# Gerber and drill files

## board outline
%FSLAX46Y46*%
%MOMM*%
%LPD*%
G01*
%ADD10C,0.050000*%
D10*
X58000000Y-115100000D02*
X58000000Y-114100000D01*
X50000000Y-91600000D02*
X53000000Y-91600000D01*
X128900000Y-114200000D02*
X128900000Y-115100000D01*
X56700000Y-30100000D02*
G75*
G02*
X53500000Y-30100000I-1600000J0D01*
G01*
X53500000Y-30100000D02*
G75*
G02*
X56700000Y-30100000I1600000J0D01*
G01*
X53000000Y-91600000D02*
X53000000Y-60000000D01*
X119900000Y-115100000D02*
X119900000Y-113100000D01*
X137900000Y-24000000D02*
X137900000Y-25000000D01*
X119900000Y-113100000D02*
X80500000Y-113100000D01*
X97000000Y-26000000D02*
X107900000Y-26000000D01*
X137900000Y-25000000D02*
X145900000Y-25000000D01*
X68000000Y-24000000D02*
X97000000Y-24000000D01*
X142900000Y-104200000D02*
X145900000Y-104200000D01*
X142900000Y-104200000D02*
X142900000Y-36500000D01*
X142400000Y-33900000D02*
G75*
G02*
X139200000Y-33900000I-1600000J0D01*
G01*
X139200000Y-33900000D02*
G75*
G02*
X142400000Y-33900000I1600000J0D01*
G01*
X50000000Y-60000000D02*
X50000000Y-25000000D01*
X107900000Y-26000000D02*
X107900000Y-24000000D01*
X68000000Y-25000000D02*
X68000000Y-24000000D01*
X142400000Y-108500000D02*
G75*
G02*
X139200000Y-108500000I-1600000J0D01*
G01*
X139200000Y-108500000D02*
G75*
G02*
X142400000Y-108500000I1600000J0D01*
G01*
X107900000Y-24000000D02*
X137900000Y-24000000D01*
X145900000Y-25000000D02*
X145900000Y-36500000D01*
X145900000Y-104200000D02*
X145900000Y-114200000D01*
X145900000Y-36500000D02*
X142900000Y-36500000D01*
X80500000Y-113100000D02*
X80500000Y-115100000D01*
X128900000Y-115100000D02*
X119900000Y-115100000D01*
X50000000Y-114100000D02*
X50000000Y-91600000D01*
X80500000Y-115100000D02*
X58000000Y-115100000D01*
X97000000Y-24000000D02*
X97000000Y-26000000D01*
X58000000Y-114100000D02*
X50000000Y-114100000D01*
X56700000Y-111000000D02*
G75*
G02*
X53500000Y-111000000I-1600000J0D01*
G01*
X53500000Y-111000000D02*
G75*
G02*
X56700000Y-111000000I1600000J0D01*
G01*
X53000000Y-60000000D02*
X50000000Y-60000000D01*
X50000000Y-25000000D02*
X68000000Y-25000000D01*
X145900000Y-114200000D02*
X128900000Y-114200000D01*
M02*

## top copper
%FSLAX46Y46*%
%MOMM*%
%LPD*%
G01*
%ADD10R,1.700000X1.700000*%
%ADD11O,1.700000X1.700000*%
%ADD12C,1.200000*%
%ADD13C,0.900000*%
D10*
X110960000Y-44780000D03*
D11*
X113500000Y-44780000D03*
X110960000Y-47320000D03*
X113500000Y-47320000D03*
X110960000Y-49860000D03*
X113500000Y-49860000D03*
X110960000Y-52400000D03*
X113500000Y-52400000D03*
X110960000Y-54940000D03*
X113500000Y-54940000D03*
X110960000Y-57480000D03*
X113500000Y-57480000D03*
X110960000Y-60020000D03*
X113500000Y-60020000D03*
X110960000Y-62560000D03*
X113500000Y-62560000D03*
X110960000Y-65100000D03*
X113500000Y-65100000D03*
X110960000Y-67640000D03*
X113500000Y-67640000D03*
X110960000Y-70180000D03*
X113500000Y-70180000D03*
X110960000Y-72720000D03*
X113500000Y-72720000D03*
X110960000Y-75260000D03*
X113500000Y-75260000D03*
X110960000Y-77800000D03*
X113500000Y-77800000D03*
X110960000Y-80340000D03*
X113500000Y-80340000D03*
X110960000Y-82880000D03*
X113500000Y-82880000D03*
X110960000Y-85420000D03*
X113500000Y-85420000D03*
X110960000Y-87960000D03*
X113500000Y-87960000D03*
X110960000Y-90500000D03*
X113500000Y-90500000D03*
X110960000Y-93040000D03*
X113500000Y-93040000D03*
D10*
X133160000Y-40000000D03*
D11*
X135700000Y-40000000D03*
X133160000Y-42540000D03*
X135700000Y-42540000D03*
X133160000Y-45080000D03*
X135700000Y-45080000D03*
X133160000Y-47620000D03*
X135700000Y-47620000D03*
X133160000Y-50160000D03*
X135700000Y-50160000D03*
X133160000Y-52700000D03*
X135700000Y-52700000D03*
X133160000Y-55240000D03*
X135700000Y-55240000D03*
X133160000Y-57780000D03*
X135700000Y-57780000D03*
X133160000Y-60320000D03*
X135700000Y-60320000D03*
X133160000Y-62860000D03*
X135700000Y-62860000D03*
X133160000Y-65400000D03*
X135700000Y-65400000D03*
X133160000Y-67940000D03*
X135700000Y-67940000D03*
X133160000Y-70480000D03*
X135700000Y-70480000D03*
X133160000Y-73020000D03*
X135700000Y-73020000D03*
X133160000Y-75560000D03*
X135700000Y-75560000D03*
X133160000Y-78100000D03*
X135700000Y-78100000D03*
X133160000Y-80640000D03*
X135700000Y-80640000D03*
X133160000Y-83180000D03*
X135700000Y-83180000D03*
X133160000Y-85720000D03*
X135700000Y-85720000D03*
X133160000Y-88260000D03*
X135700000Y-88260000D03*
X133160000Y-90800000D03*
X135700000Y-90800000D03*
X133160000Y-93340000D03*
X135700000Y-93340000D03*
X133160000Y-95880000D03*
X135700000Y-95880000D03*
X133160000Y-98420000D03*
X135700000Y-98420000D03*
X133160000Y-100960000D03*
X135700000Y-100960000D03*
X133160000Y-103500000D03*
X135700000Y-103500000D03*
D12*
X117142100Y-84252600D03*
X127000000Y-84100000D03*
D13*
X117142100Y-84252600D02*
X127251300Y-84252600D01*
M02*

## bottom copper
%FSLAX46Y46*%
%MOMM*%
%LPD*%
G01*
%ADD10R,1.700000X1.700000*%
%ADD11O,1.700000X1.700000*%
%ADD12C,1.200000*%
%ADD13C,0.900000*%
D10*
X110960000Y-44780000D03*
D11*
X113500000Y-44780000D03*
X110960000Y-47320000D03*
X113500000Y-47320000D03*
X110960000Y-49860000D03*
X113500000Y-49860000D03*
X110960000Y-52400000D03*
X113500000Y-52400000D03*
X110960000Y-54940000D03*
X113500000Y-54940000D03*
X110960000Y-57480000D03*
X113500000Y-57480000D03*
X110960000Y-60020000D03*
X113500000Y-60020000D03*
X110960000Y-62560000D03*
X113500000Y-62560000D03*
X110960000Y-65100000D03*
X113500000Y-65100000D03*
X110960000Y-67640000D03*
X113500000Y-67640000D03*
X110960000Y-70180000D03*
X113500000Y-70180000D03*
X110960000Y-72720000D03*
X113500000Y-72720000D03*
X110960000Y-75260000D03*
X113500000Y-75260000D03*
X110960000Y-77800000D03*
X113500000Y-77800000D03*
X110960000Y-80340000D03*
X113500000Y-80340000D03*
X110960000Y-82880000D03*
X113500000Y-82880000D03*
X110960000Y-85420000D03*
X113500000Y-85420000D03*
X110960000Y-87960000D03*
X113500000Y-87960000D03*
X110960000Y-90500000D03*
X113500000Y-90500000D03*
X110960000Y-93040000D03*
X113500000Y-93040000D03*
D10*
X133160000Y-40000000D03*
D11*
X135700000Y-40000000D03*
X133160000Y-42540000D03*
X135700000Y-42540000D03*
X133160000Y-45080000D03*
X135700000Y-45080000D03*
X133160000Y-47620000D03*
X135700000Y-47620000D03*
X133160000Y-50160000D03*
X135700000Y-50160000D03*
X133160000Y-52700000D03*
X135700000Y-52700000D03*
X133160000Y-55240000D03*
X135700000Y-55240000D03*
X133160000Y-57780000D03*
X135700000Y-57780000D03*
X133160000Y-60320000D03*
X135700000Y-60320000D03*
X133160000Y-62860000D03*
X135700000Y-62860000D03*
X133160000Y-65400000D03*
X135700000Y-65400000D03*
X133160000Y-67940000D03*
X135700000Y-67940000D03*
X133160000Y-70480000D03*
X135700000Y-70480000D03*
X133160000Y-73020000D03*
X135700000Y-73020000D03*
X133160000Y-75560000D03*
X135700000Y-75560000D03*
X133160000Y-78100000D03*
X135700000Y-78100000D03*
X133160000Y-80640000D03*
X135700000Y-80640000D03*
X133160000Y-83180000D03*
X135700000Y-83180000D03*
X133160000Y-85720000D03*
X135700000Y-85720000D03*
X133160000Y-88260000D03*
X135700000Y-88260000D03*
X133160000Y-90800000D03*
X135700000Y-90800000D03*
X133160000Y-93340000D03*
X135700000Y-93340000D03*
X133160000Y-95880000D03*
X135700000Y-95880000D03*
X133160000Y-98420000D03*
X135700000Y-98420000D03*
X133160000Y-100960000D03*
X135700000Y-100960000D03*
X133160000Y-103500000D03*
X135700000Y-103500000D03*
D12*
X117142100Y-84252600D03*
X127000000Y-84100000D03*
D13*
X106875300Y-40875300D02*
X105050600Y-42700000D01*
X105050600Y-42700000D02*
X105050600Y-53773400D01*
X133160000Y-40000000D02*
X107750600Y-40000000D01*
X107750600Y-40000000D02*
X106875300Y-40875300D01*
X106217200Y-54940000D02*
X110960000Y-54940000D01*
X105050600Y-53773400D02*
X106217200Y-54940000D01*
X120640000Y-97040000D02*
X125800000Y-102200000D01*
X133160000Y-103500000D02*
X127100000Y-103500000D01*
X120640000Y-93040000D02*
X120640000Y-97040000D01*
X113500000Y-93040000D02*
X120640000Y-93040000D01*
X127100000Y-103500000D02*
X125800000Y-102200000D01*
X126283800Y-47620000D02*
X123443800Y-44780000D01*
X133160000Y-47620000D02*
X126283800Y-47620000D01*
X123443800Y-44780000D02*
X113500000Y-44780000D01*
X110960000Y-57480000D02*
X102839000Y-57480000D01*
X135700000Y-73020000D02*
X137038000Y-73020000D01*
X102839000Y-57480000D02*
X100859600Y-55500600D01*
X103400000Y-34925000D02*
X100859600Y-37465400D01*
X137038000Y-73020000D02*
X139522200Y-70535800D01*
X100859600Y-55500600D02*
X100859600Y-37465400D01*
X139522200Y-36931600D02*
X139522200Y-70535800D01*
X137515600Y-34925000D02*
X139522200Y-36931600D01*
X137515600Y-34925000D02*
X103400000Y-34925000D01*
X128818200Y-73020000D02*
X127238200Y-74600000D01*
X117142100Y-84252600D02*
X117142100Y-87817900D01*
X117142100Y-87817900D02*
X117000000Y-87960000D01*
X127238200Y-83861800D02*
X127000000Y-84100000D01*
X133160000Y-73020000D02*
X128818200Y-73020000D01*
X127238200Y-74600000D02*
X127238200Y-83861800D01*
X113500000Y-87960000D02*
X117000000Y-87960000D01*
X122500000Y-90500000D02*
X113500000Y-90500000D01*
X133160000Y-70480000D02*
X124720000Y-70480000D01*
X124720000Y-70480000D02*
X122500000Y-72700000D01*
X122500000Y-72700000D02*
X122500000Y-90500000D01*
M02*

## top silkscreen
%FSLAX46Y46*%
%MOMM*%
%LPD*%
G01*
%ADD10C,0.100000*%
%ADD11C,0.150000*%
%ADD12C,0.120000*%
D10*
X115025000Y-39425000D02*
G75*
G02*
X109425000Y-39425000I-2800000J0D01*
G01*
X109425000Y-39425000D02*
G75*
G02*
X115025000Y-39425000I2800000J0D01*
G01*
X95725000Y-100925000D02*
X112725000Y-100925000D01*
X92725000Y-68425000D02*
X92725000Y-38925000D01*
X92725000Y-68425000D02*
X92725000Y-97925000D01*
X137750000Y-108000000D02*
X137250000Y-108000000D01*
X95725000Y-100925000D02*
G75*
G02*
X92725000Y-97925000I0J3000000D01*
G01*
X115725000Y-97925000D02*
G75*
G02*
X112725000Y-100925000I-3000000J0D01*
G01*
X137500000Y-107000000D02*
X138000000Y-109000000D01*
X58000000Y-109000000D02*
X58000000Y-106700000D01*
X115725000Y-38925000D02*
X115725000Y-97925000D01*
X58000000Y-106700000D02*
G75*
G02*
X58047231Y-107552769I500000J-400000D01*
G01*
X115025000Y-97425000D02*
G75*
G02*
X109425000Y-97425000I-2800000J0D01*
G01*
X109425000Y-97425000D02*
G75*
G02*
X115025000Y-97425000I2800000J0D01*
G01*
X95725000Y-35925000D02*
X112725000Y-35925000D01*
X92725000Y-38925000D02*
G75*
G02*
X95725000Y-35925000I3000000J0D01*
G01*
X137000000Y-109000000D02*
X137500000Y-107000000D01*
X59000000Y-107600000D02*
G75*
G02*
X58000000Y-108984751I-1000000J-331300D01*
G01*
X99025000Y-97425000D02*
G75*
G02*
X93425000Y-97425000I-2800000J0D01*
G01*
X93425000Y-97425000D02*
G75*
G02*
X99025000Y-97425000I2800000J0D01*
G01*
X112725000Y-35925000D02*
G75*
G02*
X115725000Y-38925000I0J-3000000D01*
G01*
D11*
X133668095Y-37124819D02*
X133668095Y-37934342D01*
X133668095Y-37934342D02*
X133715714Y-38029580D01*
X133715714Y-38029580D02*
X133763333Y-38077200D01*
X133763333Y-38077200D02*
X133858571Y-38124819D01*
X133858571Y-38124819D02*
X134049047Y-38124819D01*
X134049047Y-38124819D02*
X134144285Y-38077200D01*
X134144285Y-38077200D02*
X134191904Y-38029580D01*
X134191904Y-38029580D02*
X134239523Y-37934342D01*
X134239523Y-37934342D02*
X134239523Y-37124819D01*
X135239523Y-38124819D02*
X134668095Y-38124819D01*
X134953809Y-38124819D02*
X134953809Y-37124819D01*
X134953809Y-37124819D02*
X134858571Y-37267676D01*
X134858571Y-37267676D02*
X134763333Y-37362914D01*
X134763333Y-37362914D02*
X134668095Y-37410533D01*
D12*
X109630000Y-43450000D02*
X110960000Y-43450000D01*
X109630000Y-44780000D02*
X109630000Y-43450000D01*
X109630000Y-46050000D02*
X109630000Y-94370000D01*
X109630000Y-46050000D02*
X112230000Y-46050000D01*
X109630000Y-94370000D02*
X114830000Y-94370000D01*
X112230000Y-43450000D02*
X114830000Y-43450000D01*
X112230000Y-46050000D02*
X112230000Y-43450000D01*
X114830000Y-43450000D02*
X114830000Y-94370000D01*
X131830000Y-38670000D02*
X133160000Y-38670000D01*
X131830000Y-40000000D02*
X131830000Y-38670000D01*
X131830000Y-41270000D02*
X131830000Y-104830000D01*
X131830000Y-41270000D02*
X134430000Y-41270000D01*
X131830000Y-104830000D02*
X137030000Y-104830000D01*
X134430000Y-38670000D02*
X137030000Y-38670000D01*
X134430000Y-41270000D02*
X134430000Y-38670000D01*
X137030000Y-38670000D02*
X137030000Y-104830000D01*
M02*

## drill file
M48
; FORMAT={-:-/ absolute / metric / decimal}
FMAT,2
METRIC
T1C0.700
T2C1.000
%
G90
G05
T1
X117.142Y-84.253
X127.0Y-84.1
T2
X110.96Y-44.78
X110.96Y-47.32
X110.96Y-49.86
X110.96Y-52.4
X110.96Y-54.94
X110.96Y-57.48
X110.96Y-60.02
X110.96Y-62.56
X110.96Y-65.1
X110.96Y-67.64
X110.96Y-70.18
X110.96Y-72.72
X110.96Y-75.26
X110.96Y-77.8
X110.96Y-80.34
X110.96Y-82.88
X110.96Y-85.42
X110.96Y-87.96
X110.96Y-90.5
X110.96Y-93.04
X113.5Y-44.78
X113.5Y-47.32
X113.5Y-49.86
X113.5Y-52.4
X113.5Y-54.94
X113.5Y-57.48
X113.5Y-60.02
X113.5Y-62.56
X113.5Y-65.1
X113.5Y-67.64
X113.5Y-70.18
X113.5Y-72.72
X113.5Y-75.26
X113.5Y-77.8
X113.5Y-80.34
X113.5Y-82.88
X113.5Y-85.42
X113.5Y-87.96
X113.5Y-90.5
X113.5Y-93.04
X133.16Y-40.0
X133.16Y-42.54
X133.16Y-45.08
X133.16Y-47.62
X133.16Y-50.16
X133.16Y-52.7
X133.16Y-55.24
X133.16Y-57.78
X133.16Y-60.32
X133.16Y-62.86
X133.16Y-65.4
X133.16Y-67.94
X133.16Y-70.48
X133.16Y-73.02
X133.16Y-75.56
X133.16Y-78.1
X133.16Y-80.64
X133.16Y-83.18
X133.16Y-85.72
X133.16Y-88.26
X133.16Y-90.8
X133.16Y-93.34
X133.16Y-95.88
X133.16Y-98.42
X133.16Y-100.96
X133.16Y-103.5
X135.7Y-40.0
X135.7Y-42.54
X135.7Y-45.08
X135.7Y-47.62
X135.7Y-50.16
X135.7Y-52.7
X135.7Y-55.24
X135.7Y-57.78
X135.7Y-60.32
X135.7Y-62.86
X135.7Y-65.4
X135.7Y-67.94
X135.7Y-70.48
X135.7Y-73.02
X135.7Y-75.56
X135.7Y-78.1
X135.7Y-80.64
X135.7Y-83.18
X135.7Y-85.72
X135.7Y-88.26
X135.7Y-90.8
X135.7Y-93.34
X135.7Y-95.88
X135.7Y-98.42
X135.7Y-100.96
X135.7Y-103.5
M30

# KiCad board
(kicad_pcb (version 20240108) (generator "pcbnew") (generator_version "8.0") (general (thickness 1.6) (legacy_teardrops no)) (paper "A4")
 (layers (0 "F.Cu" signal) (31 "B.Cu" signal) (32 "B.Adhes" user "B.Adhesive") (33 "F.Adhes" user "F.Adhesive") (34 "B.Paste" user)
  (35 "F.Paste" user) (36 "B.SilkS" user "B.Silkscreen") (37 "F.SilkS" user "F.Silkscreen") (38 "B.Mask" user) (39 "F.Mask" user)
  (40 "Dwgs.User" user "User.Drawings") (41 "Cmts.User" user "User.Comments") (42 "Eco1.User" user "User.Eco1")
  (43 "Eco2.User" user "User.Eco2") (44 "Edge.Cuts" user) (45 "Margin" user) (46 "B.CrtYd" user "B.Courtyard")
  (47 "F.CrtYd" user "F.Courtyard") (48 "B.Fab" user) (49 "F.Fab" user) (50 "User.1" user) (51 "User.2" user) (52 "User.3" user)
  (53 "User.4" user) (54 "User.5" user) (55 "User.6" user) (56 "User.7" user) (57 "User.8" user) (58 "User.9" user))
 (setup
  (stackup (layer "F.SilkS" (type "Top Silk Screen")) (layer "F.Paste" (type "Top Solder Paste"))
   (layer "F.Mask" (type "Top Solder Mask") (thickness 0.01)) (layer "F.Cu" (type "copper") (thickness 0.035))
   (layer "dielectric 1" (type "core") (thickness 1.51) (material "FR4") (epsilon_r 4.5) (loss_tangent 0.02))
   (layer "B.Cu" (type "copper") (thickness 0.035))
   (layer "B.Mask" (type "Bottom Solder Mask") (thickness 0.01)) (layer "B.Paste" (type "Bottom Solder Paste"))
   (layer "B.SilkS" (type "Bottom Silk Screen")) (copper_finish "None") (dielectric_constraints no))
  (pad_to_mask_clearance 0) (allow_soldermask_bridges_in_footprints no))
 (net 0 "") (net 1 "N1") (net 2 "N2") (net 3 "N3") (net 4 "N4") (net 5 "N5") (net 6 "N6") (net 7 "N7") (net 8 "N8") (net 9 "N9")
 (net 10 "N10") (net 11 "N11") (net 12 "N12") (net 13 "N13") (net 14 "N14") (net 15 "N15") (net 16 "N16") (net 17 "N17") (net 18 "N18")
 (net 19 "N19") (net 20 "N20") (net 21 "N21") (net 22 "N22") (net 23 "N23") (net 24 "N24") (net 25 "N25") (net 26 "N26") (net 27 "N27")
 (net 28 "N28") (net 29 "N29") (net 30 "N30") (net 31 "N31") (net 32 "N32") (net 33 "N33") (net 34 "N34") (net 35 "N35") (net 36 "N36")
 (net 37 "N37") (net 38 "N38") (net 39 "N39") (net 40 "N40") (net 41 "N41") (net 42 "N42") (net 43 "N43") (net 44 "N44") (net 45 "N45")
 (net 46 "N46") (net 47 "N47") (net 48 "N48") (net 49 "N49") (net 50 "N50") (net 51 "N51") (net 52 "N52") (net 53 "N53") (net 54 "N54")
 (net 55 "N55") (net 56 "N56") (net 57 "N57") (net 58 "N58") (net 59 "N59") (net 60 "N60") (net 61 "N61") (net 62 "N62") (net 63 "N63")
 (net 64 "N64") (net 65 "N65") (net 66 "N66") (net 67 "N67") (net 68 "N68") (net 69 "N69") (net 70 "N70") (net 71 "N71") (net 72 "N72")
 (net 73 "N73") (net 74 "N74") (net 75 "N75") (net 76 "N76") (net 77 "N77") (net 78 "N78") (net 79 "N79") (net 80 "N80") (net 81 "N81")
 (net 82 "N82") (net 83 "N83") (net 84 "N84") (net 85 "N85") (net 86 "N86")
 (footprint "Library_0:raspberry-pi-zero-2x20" (layer "F.Cu") (at 110.96 44.78)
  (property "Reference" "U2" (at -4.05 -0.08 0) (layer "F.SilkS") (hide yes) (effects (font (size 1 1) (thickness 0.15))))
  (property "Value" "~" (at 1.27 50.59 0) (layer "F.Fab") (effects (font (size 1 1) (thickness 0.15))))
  (fp_line (start -1.33 -1.33) (end 0 -1.33) (stroke (width 0.12) (type solid)) (layer "F.SilkS"))
  (fp_line (start -1.33 0) (end -1.33 -1.33) (stroke (width 0.12) (type solid)) (layer "F.SilkS"))
  (fp_line (start -1.33 1.27) (end -1.33 49.59) (stroke (width 0.12) (type solid)) (layer "F.SilkS"))
  (fp_line (start -1.33 1.27) (end 1.27 1.27) (stroke (width 0.12) (type solid)) (layer "F.SilkS"))
  (fp_line (start -1.33 49.59) (end 3.87 49.59) (stroke (width 0.12) (type solid)) (layer "F.SilkS"))
  (fp_line (start 1.27 -1.33) (end 3.87 -1.33) (stroke (width 0.12) (type solid)) (layer "F.SilkS"))
  (fp_line (start 1.27 1.27) (end 1.27 -1.33) (stroke (width 0.12) (type solid)) (layer "F.SilkS"))
  (fp_line (start 3.87 -1.33) (end 3.87 49.59) (stroke (width 0.12) (type solid)) (layer "F.SilkS"))
  (pad "1" thru_hole rect (at 0 0) (size 1.7 1.7) (drill 1) (layers "*.Cu" "*.Mask") (remove_unused_layers no) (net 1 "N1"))
  (pad "2" thru_hole oval (at 2.54 0) (size 1.7 1.7) (drill 1) (layers "*.Cu" "*.Mask") (remove_unused_layers no) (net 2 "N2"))
  (pad "3" thru_hole oval (at 0 2.54) (size 1.7 1.7) (drill 1) (layers "*.Cu" "*.Mask") (remove_unused_layers no) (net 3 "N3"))
  (pad "4" thru_hole oval (at 2.54 2.54) (size 1.7 1.7) (drill 1) (layers "*.Cu" "*.Mask") (remove_unused_layers no) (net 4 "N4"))
  (pad "5" thru_hole oval (at 0 5.08) (size 1.7 1.7) (drill 1) (layers "*.Cu" "*.Mask") (remove_unused_layers no) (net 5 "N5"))
  (pad "6" thru_hole oval (at 2.54 5.08) (size 1.7 1.7) (drill 1) (layers "*.Cu" "*.Mask") (remove_unused_layers no) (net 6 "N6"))
  (pad "7" thru_hole oval (at 0 7.62) (size 1.7 1.7) (drill 1) (layers "*.Cu" "*.Mask") (remove_unused_layers no) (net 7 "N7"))
  (pad "8" thru_hole oval (at 2.54 7.62) (size 1.7 1.7) (drill 1) (layers "*.Cu" "*.Mask") (remove_unused_layers no) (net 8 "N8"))
  (pad "9" thru_hole oval (at 0 10.16) (size 1.7 1.7) (drill 1) (layers "*.Cu" "*.Mask") (remove_unused_layers no) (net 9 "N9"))
  (pad "10" thru_hole oval (at 2.54 10.16) (size 1.7 1.7) (drill 1) (layers "*.Cu" "*.Mask") (remove_unused_layers no) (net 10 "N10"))
  (pad "11" thru_hole oval (at 0 12.7) (size 1.7 1.7) (drill 1) (layers "*.Cu" "*.Mask") (remove_unused_layers no) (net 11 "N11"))
  (pad "12" thru_hole oval (at 2.54 12.7) (size 1.7 1.7) (drill 1) (layers "*.Cu" "*.Mask") (remove_unused_layers no) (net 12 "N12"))
  (pad "13" thru_hole oval (at 0 15.24) (size 1.7 1.7) (drill 1) (layers "*.Cu" "*.Mask") (remove_unused_layers no) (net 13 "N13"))
  (pad "14" thru_hole oval (at 2.54 15.24) (size 1.7 1.7) (drill 1) (layers "*.Cu" "*.Mask") (remove_unused_layers no) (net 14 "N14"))
  (pad "15" thru_hole oval (at 0 17.78) (size 1.7 1.7) (drill 1) (layers "*.Cu" "*.Mask") (remove_unused_layers no) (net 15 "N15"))
  (pad "16" thru_hole oval (at 2.54 17.78) (size 1.7 1.7) (drill 1) (layers "*.Cu" "*.Mask") (remove_unused_layers no) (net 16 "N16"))
  (pad "17" thru_hole oval (at 0 20.32) (size 1.7 1.7) (drill 1) (layers "*.Cu" "*.Mask") (remove_unused_layers no) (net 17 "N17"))
  (pad "18" thru_hole oval (at 2.54 20.32) (size 1.7 1.7) (drill 1) (layers "*.Cu" "*.Mask") (remove_unused_layers no) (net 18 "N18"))
  (pad "19" thru_hole oval (at 0 22.86) (size 1.7 1.7) (drill 1) (layers "*.Cu" "*.Mask") (remove_unused_layers no) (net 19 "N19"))
  (pad "20" thru_hole oval (at 2.54 22.86) (size 1.7 1.7) (drill 1) (layers "*.Cu" "*.Mask") (remove_unused_layers no) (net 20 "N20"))
  (pad "21" thru_hole oval (at 0 25.4) (size 1.7 1.7) (drill 1) (layers "*.Cu" "*.Mask") (remove_unused_layers no) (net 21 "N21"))
  (pad "22" thru_hole oval (at 2.54 25.4) (size 1.7 1.7) (drill 1) (layers "*.Cu" "*.Mask") (remove_unused_layers no) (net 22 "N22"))
  (pad "23" thru_hole oval (at 0 27.94) (size 1.7 1.7) (drill 1) (layers "*.Cu" "*.Mask") (remove_unused_layers no) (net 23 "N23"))
  (pad "24" thru_hole oval (at 2.54 27.94) (size 1.7 1.7) (drill 1) (layers "*.Cu" "*.Mask") (remove_unused_layers no) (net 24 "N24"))
  (pad "25" thru_hole oval (at 0 30.48) (size 1.7 1.7) (drill 1) (layers "*.Cu" "*.Mask") (remove_unused_layers no) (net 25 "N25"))
  (pad "26" thru_hole oval (at 2.54 30.48) (size 1.7 1.7) (drill 1) (layers "*.Cu" "*.Mask") (remove_unused_layers no) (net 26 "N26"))
  (pad "27" thru_hole oval (at 0 33.02) (size 1.7 1.7) (drill 1) (layers "*.Cu" "*.Mask") (remove_unused_layers no) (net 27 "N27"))
  (pad "28" thru_hole oval (at 2.54 33.02) (size 1.7 1.7) (drill 1) (layers "*.Cu" "*.Mask") (remove_unused_layers no) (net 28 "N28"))
  (pad "29" thru_hole oval (at 0 35.56) (size 1.7 1.7) (drill 1) (layers "*.Cu" "*.Mask") (remove_unused_layers no) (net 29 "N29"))
  (pad "30" thru_hole oval (at 2.54 35.56) (size 1.7 1.7) (drill 1) (layers "*.Cu" "*.Mask") (remove_unused_layers no) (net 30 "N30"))
  (pad "31" thru_hole oval (at 0 38.1) (size 1.7 1.7) (drill 1) (layers "*.Cu" "*.Mask") (remove_unused_layers no) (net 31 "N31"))
  (pad "32" thru_hole oval (at 2.54 38.1) (size 1.7 1.7) (drill 1) (layers "*.Cu" "*.Mask") (remove_unused_layers no) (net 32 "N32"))
  (pad "33" thru_hole oval (at 0 40.64) (size 1.7 1.7) (drill 1) (layers "*.Cu" "*.Mask") (remove_unused_layers no) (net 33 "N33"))
  (pad "34" thru_hole oval (at 2.54 40.64) (size 1.7 1.7) (drill 1) (layers "*.Cu" "*.Mask") (remove_unused_layers no) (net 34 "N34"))
  (pad "35" thru_hole oval (at 0 43.18) (size 1.7 1.7) (drill 1) (layers "*.Cu" "*.Mask") (remove_unused_layers no) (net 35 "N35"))
  (pad "36" thru_hole oval (at 2.54 43.18) (size 1.7 1.7) (drill 1) (layers "*.Cu" "*.Mask") (remove_unused_layers no) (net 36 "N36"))
  (pad "37" thru_hole oval (at 0 45.72) (size 1.7 1.7) (drill 1) (layers "*.Cu" "*.Mask") (remove_unused_layers no) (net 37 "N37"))
  (pad "38" thru_hole oval (at 2.54 45.72) (size 1.7 1.7) (drill 1) (layers "*.Cu" "*.Mask") (remove_unused_layers no) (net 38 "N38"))
  (pad "39" thru_hole oval (at 0 48.26) (size 1.7 1.7) (drill 1) (layers "*.Cu" "*.Mask") (remove_unused_layers no) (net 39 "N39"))
  (pad "40" thru_hole oval (at 2.54 48.26) (size 1.7 1.7) (drill 1) (layers "*.Cu" "*.Mask") (remove_unused_layers no) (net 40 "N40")))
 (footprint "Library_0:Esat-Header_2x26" (layer "F.Cu") (at 133.16 40)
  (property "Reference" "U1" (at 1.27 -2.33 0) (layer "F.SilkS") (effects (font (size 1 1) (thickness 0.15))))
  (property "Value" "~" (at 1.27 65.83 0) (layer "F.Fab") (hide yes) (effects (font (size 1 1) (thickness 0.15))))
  (fp_line (start -1.33 -1.33) (end 0 -1.33) (stroke (width 0.12) (type solid)) (layer "F.SilkS"))
  (fp_line (start -1.33 0) (end -1.33 -1.33) (stroke (width 0.12) (type solid)) (layer "F.SilkS"))
  (fp_line (start -1.33 1.27) (end -1.33 64.83) (stroke (width 0.12) (type solid)) (layer "F.SilkS"))
  (fp_line (start -1.33 1.27) (end 1.27 1.27) (stroke (width 0.12) (type solid)) (layer "F.SilkS"))
  (fp_line (start -1.33 64.83) (end 3.87 64.83) (stroke (width 0.12) (type solid)) (layer "F.SilkS"))
  (fp_line (start 1.27 -1.33) (end 3.87 -1.33) (stroke (width 0.12) (type solid)) (layer "F.SilkS"))
  (fp_line (start 1.27 1.27) (end 1.27 -1.33) (stroke (width 0.12) (type solid)) (layer "F.SilkS"))
  (fp_line (start 3.87 -1.33) (end 3.87 64.83) (stroke (width 0.12) (type solid)) (layer "F.SilkS"))
  (pad "1" thru_hole rect (at 0 0) (size 1.7 1.7) (drill 1) (layers "*.Cu" "*.Mask") (remove_unused_layers no) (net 9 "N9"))
  (pad "2" thru_hole oval (at 2.54 0) (size 1.7 1.7) (drill 1) (layers "*.Cu" "*.Mask") (remove_unused_layers no) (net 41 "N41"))
  (pad "3" thru_hole oval (at 0 2.54) (size 1.7 1.7) (drill 1) (layers "*.Cu" "*.Mask") (remove_unused_layers no) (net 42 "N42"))
  (pad "4" thru_hole oval (at 2.54 2.54) (size 1.7 1.7) (drill 1) (layers "*.Cu" "*.Mask") (remove_unused_layers no) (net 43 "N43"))
  (pad "5" thru_hole oval (at 0 5.08) (size 1.7 1.7) (drill 1) (layers "*.Cu" "*.Mask") (remove_unused_layers no) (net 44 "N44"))
  (pad "6" thru_hole oval (at 2.54 5.08) (size 1.7 1.7) (drill 1) (layers "*.Cu" "*.Mask") (remove_unused_layers no) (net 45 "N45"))
  (pad "7" thru_hole oval (at 0 7.62) (size 1.7 1.7) (drill 1) (layers "*.Cu" "*.Mask") (remove_unused_layers no) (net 2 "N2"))
  (pad "8" thru_hole oval (at 2.54 7.62) (size 1.7 1.7) (drill 1) (layers "*.Cu" "*.Mask") (remove_unused_layers no) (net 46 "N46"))
  (pad "9" thru_hole oval (at 0 10.16) (size 1.7 1.7) (drill 1) (layers "*.Cu" "*.Mask") (remove_unused_layers no) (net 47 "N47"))
  (pad "10" thru_hole oval (at 2.54 10.16) (size 1.7 1.7) (drill 1) (layers "*.Cu" "*.Mask") (remove_unused_layers no) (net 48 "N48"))
  (pad "11" thru_hole oval (at 0 12.7) (size 1.7 1.7) (drill 1) (layers "*.Cu" "*.Mask") (remove_unused_layers no) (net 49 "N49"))
  (pad "12" thru_hole oval (at 2.54 12.7) (size 1.7 1.7) (drill 1) (layers "*.Cu" "*.Mask") (remove_unused_layers no) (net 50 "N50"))
  (pad "13" thru_hole oval (at 0 15.24) (size 1.7 1.7) (drill 1) (layers "*.Cu" "*.Mask") (remove_unused_layers no) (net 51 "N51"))
  (pad "14" thru_hole oval (at 2.54 15.24) (size 1.7 1.7) (drill 1) (layers "*.Cu" "*.Mask") (remove_unused_layers no) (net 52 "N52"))
  (pad "15" thru_hole oval (at 0 17.78) (size 1.7 1.7) (drill 1) (layers "*.Cu" "*.Mask") (remove_unused_layers no) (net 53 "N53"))
  (pad "16" thru_hole oval (at 2.54 17.78) (size 1.7 1.7) (drill 1) (layers "*.Cu" "*.Mask") (remove_unused_layers no) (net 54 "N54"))
  (pad "17" thru_hole oval (at 0 20.32) (size 1.7 1.7) (drill 1) (layers "*.Cu" "*.Mask") (remove_unused_layers no) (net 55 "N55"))
  (pad "18" thru_hole oval (at 2.54 20.32) (size 1.7 1.7) (drill 1) (layers "*.Cu" "*.Mask") (remove_unused_layers no) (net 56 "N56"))
  (pad "19" thru_hole oval (at 0 22.86) (size 1.7 1.7) (drill 1) (layers "*.Cu" "*.Mask") (remove_unused_layers no) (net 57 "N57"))
  (pad "20" thru_hole oval (at 2.54 22.86) (size 1.7 1.7) (drill 1) (layers "*.Cu" "*.Mask") (remove_unused_layers no) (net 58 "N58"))
  (pad "21" thru_hole oval (at 0 25.4) (size 1.7 1.7) (drill 1) (layers "*.Cu" "*.Mask") (remove_unused_layers no) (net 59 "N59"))
  (pad "22" thru_hole oval (at 2.54 25.4) (size 1.7 1.7) (drill 1) (layers "*.Cu" "*.Mask") (remove_unused_layers no) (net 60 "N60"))
  (pad "23" thru_hole oval (at 0 27.94) (size 1.7 1.7) (drill 1) (layers "*.Cu" "*.Mask") (remove_unused_layers no) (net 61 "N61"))
  (pad "24" thru_hole oval (at 2.54 27.94) (size 1.7 1.7) (drill 1) (layers "*.Cu" "*.Mask") (remove_unused_layers no) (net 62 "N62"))
  (pad "25" thru_hole oval (at 0 30.48) (size 1.7 1.7) (drill 1) (layers "*.Cu" "*.Mask") (remove_unused_layers no) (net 38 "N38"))
  (pad "26" thru_hole oval (at 2.54 30.48) (size 1.7 1.7) (drill 1) (layers "*.Cu" "*.Mask") (remove_unused_layers no) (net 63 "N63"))
  (pad "27" thru_hole oval (at 0 33.02) (size 1.7 1.7) (drill 1) (layers "*.Cu" "*.Mask") (remove_unused_layers no) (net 36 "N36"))
  (pad "28" thru_hole oval (at 2.54 33.02) (size 1.7 1.7) (drill 1) (layers "*.Cu" "*.Mask") (remove_unused_layers no) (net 11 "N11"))
  (pad "29" thru_hole oval (at 0 35.56) (size 1.7 1.7) (drill 1) (layers "*.Cu" "*.Mask") (remove_unused_layers no) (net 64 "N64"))
  (pad "30" thru_hole oval (at 2.54 35.56) (size 1.7 1.7) (drill 1) (layers "*.Cu" "*.Mask") (remove_unused_layers no) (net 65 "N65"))
  (pad "31" thru_hole oval (at 0 38.1) (size 1.7 1.7) (drill 1) (layers "*.Cu" "*.Mask") (remove_unused_layers no) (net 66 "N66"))
  (pad "32" thru_hole oval (at 2.54 38.1) (size 1.7 1.7) (drill 1) (layers "*.Cu" "*.Mask") (remove_unused_layers no) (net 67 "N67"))
  (pad "33" thru_hole oval (at 0 40.64) (size 1.7 1.7) (drill 1) (layers "*.Cu" "*.Mask") (remove_unused_layers no) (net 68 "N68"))
  (pad "34" thru_hole oval (at 2.54 40.64) (size 1.7 1.7) (drill 1) (layers "*.Cu" "*.Mask") (remove_unused_layers no) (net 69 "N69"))
  (pad "35" thru_hole oval (at 0 43.18) (size 1.7 1.7) (drill 1) (layers "*.Cu" "*.Mask") (remove_unused_layers no) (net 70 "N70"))
  (pad "36" thru_hole oval (at 2.54 43.18) (size 1.7 1.7) (drill 1) (layers "*.Cu" "*.Mask") (remove_unused_layers no) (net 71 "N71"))
  (pad "37" thru_hole oval (at 0 45.72) (size 1.7 1.7) (drill 1) (layers "*.Cu" "*.Mask") (remove_unused_layers no) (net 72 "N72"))
  (pad "38" thru_hole oval (at 2.54 45.72) (size 1.7 1.7) (drill 1) (layers "*.Cu" "*.Mask") (remove_unused_layers no) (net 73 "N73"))
  (pad "39" thru_hole oval (at 0 48.26) (size 1.7 1.7) (drill 1) (layers "*.Cu" "*.Mask") (remove_unused_layers no) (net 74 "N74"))
  (pad "40" thru_hole oval (at 2.54 48.26) (size 1.7 1.7) (drill 1) (layers "*.Cu" "*.Mask") (remove_unused_layers no) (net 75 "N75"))
  (pad "41" thru_hole oval (at 0 50.8) (size 1.7 1.7) (drill 1) (layers "*.Cu" "*.Mask") (remove_unused_layers no) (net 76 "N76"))
  (pad "42" thru_hole oval (at 2.54 50.8) (size 1.7 1.7) (drill 1) (layers "*.Cu" "*.Mask") (remove_unused_layers no) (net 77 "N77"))
  (pad "43" thru_hole oval (at 0 53.34) (size 1.7 1.7) (drill 1) (layers "*.Cu" "*.Mask") (remove_unused_layers no) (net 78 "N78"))
  (pad "44" thru_hole oval (at 2.54 53.34) (size 1.7 1.7) (drill 1) (layers "*.Cu" "*.Mask") (remove_unused_layers no) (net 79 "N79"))
  (pad "45" thru_hole oval (at 0 55.88) (size 1.7 1.7) (drill 1) (layers "*.Cu" "*.Mask") (remove_unused_layers no) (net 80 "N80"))
  (pad "46" thru_hole oval (at 2.54 55.88) (size 1.7 1.7) (drill 1) (layers "*.Cu" "*.Mask") (remove_unused_layers no) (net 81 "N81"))
  (pad "47" thru_hole oval (at 0 58.42) (size 1.7 1.7) (drill 1) (layers "*.Cu" "*.Mask") (remove_unused_layers no) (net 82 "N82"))
  (pad "48" thru_hole oval (at 2.54 58.42) (size 1.7 1.7) (drill 1) (layers "*.Cu" "*.Mask") (remove_unused_layers no) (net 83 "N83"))
  (pad "49" thru_hole oval (at 0 60.96) (size 1.7 1.7) (drill 1) (layers "*.Cu" "*.Mask") (remove_unused_layers no) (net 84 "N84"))
  (pad "50" thru_hole oval (at 2.54 60.96) (size 1.7 1.7) (drill 1) (layers "*.Cu" "*.Mask") (remove_unused_layers no) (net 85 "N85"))
  (pad "51" thru_hole oval (at 0 63.5) (size 1.7 1.7) (drill 1) (layers "*.Cu" "*.Mask") (remove_unused_layers no) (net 40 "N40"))
  (pad "52" thru_hole oval (at 2.54 63.5) (size 1.7 1.7) (drill 1) (layers "*.Cu" "*.Mask") (remove_unused_layers no) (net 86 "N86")))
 (gr_circle (center 112.225 39.425) (end 115.025 39.425) (stroke (width 0.1) (type default)) (fill none) (layer "F.SilkS"))
 (gr_line (start 95.725 100.925) (end 112.725 100.925) (stroke (width 0.1) (type default)) (layer "F.SilkS"))
 (gr_line (start 92.725 68.425) (end 92.725 38.925) (stroke (width 0.1) (type default)) (layer "F.SilkS"))
 (gr_line (start 92.725 68.425) (end 92.725 97.925) (stroke (width 0.1) (type default)) (layer "F.SilkS"))
 (gr_line (start 137.75 108) (end 137.25 108) (stroke (width 0.1) (type default)) (layer "F.SilkS"))
 (gr_arc (start 95.725 100.925) (mid 93.60368 100.04632) (end 92.725 97.925) (stroke (width 0.1) (type default)) (layer "F.SilkS"))
 (gr_arc (start 115.725 97.925) (mid 114.84632 100.04632) (end 112.725 100.925) (stroke (width 0.1) (type default)) (layer "F.SilkS"))
 (gr_line (start 137.5 107) (end 138 109) (stroke (width 0.1) (type default)) (layer "F.SilkS"))
 (gr_line (start 58 109) (end 58 106.7) (stroke (width 0.1) (type default)) (layer "F.SilkS"))
 (gr_line (start 115.725 38.925) (end 115.725 97.925) (stroke (width 0.1) (type default)) (layer "F.SilkS"))
 (gr_arc (start 58 106.7) (mid 59.139333 107.06459) (end 58.047231 107.552769) (stroke (width 0.1) (type default)) (layer "F.SilkS"))
 (gr_circle (center 112.225 97.425) (end 115.025 97.425) (stroke (width 0.1) (type default)) (fill none) (layer "F.SilkS"))
 (gr_line (start 95.725 35.925) (end 112.725 35.925) (stroke (width 0.1) (type default)) (layer "F.SilkS"))
 (gr_arc (start 92.725 38.925) (mid 93.60368 36.80368) (end 95.725 35.925) (stroke (width 0.1) (type default)) (layer "F.SilkS"))
 (gr_line (start 137 109) (end 137.5 107) (stroke (width 0.1) (type default)) (layer "F.SilkS"))
 (gr_arc (start 59 107.6) (mid 58.854058 108.548074) (end 58 108.984797) (stroke (width 0.1) (type default)) (layer "F.SilkS"))
 (gr_circle (center 96.225 97.425) (end 93.425 97.425) (stroke (width 0.1) (type default)) (fill none) (layer "F.SilkS"))
 (gr_arc (start 112.725 35.925) (mid 114.84632 36.80368) (end 115.725 38.925) (stroke (width 0.1) (type default)) (layer "F.SilkS"))
 (gr_line (start 58 115.1) (end 58 114.1) (stroke (width 0.05) (type default)) (layer "Edge.Cuts"))
 (gr_line (start 50 91.6) (end 53 91.6) (stroke (width 0.05) (type default)) (layer "Edge.Cuts"))
 (gr_line (start 128.9 114.2) (end 128.9 115.1) (stroke (width 0.05) (type default)) (layer "Edge.Cuts"))
 (gr_circle (center 55.1 30.1) (end 55.1 28.5) (stroke (width 0.05) (type default)) (fill none) (layer "Edge.Cuts"))
 (gr_line (start 53 91.6) (end 53 60) (stroke (width 0.05) (type default)) (layer "Edge.Cuts"))
 (gr_line (start 119.9 115.1) (end 119.9 113.1) (stroke (width 0.05) (type default)) (layer "Edge.Cuts"))
 (gr_line (start 137.9 24) (end 137.9 25) (stroke (width 0.05) (type default)) (layer "Edge.Cuts"))
 (gr_line (start 119.9 113.1) (end 80.5 113.1) (stroke (width 0.05) (type default)) (layer "Edge.Cuts"))
 (gr_line (start 97 26) (end 107.9 26) (stroke (width 0.05) (type default)) (layer "Edge.Cuts"))
 (gr_line (start 137.9 25) (end 145.9 25) (stroke (width 0.05) (type default)) (layer "Edge.Cuts"))
 (gr_line (start 68 24) (end 97 24) (stroke (width 0.05) (type default)) (layer "Edge.Cuts"))
 (gr_line (start 142.9 104.2) (end 145.9 104.2) (stroke (width 0.05) (type default)) (layer "Edge.Cuts"))
 (gr_line (start 142.9 104.2) (end 142.9 36.5) (stroke (width 0.05) (type default)) (layer "Edge.Cuts"))
 (gr_circle (center 140.8 33.9) (end 140.8 32.3) (stroke (width 0.05) (type default)) (fill none) (layer "Edge.Cuts"))
 (gr_line (start 50 60) (end 50 25) (stroke (width 0.05) (type default)) (layer "Edge.Cuts"))
 (gr_line (start 107.9 26) (end 107.9 24) (stroke (width 0.05) (type default)) (layer "Edge.Cuts"))
 (gr_line (start 68 25) (end 68 24) (stroke (width 0.05) (type default)) (layer "Edge.Cuts"))
 (gr_circle (center 140.8 108.5) (end 140.8 110.1) (stroke (width 0.05) (type default)) (fill none) (layer "Edge.Cuts"))
 (gr_line (start 107.9 24) (end 137.9 24) (stroke (width 0.05) (type default)) (layer "Edge.Cuts"))
 (gr_line (start 145.9 25) (end 145.9 36.5) (stroke (width 0.05) (type default)) (layer "Edge.Cuts"))
 (gr_line (start 145.9 104.2) (end 145.9 114.2) (stroke (width 0.05) (type default)) (layer "Edge.Cuts"))
 (gr_line (start 145.9 36.5) (end 142.9 36.5) (stroke (width 0.05) (type default)) (layer "Edge.Cuts"))
 (gr_line (start 80.5 113.1) (end 80.5 115.1) (stroke (width 0.05) (type default)) (layer "Edge.Cuts"))
 (gr_line (start 128.9 115.1) (end 119.9 115.1) (stroke (width 0.05) (type default)) (layer "Edge.Cuts"))
 (gr_line (start 50 114.1) (end 50 91.6) (stroke (width 0.05) (type default)) (layer "Edge.Cuts"))
 (gr_line (start 80.5 115.1) (end 58 115.1) (stroke (width 0.05) (type default)) (layer "Edge.Cuts"))
 (gr_line (start 97 24) (end 97 26) (stroke (width 0.05) (type default)) (layer "Edge.Cuts"))
 (gr_line (start 58 114.1) (end 50 114.1) (stroke (width 0.05) (type default)) (layer "Edge.Cuts"))
 (gr_circle (center 55.1 111) (end 55.1 109.4) (stroke (width 0.05) (type default)) (fill none) (layer "Edge.Cuts"))
 (gr_line (start 53 60) (end 50 60) (stroke (width 0.05) (type default)) (layer "Edge.Cuts"))
 (gr_line (start 50 25) (end 68 25) (stroke (width 0.05) (type default)) (layer "Edge.Cuts"))
 (gr_line (start 145.9 114.2) (end 128.9 114.2) (stroke (width 0.05) (type default)) (layer "Edge.Cuts"))
 (segment (start 106.8753 40.8753) (end 105.0506 42.7) (width 0.9) (layer "B.Cu") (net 9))
 (segment (start 105.0506 42.7) (end 105.0506 53.7734) (width 0.9) (layer "B.Cu") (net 9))
 (segment (start 133.16 40) (end 107.7506 40) (width 0.9) (layer "B.Cu") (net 9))
 (segment (start 107.7506 40) (end 106.8753 40.8753) (width 0.9) (layer "B.Cu") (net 9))
 (segment (start 106.2172 54.94) (end 110.96 54.94) (width 0.9) (layer "B.Cu") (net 9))
 (segment (start 105.0506 53.7734) (end 106.2172 54.94) (width 0.9) (layer "B.Cu") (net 9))
 (segment (start 120.64 97.04) (end 125.8 102.2) (width 0.9) (layer "B.Cu") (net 40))
 (segment (start 133.16 103.5) (end 127.1 103.5) (width 0.9) (layer "B.Cu") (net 40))
 (segment (start 120.64 93.04) (end 120.64 97.04) (width 0.9) (layer "B.Cu") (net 40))
 (segment (start 113.5 93.04) (end 120.64 93.04) (width 0.9) (layer "B.Cu") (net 40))
 (segment (start 127.1 103.5) (end 125.8 102.2) (width 0.9) (layer "B.Cu") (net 40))
 (segment (start 126.2838 47.62) (end 123.4438 44.78) (width 0.9) (layer "B.Cu") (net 2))
 (segment (start 133.16 47.62) (end 126.2838 47.62) (width 0.9) (layer "B.Cu") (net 2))
 (segment (start 123.4438 44.78) (end 113.5 44.78) (width 0.9) (layer "B.Cu") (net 2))
 (segment (start 110.96 57.48) (end 102.839 57.48) (width 0.9) (layer "B.Cu") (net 11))
 (segment (start 135.7 73.02) (end 137.038 73.02) (width 0.9) (layer "B.Cu") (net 11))
 (segment (start 102.839 57.48) (end 100.8596 55.5006) (width 0.9) (layer "B.Cu") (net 11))
 (segment (start 103.4 34.925) (end 100.8596 37.4654) (width 0.9) (layer "B.Cu") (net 11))
 (segment (start 137.038 73.02) (end 139.5222 70.5358) (width 0.9) (layer "B.Cu") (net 11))
 (segment (start 100.8596 55.5006) (end 100.8596 37.4654) (width 0.9) (layer "B.Cu") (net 11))
 (segment (start 139.5222 36.9316) (end 139.5222 70.5358) (width 0.9) (layer "B.Cu") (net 11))
 (segment (start 137.5156 34.925) (end 139.5222 36.9316) (width 0.9) (layer "B.Cu") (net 11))
 (segment (start 137.5156 34.925) (end 103.4 34.925) (width 0.9) (layer "B.Cu") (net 11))
 (segment (start 117.1421 84.2526) (end 127.2513 84.2526) (width 0.9) (layer "F.Cu") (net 36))
 (via (at 117.1421 84.2526) (size 1.2) (drill 0.7) (layers "F.Cu" "B.Cu") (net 36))
 (via (at 127 84.1) (size 1.2) (drill 0.7) (layers "F.Cu" "B.Cu") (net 36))
 (segment (start 128.8182 73.02) (end 127.2382 74.6) (width 0.9) (layer "B.Cu") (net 36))
 (segment (start 117.1421 84.2526) (end 117.1421 87.8179) (width 0.9) (layer "B.Cu") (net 36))
 (segment (start 117.1421 87.8179) (end 117 87.96) (width 0.9) (layer "B.Cu") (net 36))
 (segment (start 127.2382 83.8618) (end 127 84.1) (width 0.9) (layer "B.Cu") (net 36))
 (segment (start 133.16 73.02) (end 128.8182 73.02) (width 0.9) (layer "B.Cu") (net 36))
 (segment (start 127.2382 74.6) (end 127.2382 83.8618) (width 0.9) (layer "B.Cu") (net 36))
 (segment (start 113.5 87.96) (end 117 87.96) (width 0.9) (layer "B.Cu") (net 36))
 (segment (start 122.5 90.5) (end 113.5 90.5) (width 0.9) (layer "B.Cu") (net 38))
 (segment (start 133.16 70.48) (end 124.72 70.48) (width 0.9) (layer "B.Cu") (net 38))
 (segment (start 124.72 70.48) (end 122.5 72.7) (width 0.9) (layer "B.Cu") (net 38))
 (segment (start 122.5 72.7) (end 122.5 90.5) (width 0.9) (layer "B.Cu") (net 38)))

